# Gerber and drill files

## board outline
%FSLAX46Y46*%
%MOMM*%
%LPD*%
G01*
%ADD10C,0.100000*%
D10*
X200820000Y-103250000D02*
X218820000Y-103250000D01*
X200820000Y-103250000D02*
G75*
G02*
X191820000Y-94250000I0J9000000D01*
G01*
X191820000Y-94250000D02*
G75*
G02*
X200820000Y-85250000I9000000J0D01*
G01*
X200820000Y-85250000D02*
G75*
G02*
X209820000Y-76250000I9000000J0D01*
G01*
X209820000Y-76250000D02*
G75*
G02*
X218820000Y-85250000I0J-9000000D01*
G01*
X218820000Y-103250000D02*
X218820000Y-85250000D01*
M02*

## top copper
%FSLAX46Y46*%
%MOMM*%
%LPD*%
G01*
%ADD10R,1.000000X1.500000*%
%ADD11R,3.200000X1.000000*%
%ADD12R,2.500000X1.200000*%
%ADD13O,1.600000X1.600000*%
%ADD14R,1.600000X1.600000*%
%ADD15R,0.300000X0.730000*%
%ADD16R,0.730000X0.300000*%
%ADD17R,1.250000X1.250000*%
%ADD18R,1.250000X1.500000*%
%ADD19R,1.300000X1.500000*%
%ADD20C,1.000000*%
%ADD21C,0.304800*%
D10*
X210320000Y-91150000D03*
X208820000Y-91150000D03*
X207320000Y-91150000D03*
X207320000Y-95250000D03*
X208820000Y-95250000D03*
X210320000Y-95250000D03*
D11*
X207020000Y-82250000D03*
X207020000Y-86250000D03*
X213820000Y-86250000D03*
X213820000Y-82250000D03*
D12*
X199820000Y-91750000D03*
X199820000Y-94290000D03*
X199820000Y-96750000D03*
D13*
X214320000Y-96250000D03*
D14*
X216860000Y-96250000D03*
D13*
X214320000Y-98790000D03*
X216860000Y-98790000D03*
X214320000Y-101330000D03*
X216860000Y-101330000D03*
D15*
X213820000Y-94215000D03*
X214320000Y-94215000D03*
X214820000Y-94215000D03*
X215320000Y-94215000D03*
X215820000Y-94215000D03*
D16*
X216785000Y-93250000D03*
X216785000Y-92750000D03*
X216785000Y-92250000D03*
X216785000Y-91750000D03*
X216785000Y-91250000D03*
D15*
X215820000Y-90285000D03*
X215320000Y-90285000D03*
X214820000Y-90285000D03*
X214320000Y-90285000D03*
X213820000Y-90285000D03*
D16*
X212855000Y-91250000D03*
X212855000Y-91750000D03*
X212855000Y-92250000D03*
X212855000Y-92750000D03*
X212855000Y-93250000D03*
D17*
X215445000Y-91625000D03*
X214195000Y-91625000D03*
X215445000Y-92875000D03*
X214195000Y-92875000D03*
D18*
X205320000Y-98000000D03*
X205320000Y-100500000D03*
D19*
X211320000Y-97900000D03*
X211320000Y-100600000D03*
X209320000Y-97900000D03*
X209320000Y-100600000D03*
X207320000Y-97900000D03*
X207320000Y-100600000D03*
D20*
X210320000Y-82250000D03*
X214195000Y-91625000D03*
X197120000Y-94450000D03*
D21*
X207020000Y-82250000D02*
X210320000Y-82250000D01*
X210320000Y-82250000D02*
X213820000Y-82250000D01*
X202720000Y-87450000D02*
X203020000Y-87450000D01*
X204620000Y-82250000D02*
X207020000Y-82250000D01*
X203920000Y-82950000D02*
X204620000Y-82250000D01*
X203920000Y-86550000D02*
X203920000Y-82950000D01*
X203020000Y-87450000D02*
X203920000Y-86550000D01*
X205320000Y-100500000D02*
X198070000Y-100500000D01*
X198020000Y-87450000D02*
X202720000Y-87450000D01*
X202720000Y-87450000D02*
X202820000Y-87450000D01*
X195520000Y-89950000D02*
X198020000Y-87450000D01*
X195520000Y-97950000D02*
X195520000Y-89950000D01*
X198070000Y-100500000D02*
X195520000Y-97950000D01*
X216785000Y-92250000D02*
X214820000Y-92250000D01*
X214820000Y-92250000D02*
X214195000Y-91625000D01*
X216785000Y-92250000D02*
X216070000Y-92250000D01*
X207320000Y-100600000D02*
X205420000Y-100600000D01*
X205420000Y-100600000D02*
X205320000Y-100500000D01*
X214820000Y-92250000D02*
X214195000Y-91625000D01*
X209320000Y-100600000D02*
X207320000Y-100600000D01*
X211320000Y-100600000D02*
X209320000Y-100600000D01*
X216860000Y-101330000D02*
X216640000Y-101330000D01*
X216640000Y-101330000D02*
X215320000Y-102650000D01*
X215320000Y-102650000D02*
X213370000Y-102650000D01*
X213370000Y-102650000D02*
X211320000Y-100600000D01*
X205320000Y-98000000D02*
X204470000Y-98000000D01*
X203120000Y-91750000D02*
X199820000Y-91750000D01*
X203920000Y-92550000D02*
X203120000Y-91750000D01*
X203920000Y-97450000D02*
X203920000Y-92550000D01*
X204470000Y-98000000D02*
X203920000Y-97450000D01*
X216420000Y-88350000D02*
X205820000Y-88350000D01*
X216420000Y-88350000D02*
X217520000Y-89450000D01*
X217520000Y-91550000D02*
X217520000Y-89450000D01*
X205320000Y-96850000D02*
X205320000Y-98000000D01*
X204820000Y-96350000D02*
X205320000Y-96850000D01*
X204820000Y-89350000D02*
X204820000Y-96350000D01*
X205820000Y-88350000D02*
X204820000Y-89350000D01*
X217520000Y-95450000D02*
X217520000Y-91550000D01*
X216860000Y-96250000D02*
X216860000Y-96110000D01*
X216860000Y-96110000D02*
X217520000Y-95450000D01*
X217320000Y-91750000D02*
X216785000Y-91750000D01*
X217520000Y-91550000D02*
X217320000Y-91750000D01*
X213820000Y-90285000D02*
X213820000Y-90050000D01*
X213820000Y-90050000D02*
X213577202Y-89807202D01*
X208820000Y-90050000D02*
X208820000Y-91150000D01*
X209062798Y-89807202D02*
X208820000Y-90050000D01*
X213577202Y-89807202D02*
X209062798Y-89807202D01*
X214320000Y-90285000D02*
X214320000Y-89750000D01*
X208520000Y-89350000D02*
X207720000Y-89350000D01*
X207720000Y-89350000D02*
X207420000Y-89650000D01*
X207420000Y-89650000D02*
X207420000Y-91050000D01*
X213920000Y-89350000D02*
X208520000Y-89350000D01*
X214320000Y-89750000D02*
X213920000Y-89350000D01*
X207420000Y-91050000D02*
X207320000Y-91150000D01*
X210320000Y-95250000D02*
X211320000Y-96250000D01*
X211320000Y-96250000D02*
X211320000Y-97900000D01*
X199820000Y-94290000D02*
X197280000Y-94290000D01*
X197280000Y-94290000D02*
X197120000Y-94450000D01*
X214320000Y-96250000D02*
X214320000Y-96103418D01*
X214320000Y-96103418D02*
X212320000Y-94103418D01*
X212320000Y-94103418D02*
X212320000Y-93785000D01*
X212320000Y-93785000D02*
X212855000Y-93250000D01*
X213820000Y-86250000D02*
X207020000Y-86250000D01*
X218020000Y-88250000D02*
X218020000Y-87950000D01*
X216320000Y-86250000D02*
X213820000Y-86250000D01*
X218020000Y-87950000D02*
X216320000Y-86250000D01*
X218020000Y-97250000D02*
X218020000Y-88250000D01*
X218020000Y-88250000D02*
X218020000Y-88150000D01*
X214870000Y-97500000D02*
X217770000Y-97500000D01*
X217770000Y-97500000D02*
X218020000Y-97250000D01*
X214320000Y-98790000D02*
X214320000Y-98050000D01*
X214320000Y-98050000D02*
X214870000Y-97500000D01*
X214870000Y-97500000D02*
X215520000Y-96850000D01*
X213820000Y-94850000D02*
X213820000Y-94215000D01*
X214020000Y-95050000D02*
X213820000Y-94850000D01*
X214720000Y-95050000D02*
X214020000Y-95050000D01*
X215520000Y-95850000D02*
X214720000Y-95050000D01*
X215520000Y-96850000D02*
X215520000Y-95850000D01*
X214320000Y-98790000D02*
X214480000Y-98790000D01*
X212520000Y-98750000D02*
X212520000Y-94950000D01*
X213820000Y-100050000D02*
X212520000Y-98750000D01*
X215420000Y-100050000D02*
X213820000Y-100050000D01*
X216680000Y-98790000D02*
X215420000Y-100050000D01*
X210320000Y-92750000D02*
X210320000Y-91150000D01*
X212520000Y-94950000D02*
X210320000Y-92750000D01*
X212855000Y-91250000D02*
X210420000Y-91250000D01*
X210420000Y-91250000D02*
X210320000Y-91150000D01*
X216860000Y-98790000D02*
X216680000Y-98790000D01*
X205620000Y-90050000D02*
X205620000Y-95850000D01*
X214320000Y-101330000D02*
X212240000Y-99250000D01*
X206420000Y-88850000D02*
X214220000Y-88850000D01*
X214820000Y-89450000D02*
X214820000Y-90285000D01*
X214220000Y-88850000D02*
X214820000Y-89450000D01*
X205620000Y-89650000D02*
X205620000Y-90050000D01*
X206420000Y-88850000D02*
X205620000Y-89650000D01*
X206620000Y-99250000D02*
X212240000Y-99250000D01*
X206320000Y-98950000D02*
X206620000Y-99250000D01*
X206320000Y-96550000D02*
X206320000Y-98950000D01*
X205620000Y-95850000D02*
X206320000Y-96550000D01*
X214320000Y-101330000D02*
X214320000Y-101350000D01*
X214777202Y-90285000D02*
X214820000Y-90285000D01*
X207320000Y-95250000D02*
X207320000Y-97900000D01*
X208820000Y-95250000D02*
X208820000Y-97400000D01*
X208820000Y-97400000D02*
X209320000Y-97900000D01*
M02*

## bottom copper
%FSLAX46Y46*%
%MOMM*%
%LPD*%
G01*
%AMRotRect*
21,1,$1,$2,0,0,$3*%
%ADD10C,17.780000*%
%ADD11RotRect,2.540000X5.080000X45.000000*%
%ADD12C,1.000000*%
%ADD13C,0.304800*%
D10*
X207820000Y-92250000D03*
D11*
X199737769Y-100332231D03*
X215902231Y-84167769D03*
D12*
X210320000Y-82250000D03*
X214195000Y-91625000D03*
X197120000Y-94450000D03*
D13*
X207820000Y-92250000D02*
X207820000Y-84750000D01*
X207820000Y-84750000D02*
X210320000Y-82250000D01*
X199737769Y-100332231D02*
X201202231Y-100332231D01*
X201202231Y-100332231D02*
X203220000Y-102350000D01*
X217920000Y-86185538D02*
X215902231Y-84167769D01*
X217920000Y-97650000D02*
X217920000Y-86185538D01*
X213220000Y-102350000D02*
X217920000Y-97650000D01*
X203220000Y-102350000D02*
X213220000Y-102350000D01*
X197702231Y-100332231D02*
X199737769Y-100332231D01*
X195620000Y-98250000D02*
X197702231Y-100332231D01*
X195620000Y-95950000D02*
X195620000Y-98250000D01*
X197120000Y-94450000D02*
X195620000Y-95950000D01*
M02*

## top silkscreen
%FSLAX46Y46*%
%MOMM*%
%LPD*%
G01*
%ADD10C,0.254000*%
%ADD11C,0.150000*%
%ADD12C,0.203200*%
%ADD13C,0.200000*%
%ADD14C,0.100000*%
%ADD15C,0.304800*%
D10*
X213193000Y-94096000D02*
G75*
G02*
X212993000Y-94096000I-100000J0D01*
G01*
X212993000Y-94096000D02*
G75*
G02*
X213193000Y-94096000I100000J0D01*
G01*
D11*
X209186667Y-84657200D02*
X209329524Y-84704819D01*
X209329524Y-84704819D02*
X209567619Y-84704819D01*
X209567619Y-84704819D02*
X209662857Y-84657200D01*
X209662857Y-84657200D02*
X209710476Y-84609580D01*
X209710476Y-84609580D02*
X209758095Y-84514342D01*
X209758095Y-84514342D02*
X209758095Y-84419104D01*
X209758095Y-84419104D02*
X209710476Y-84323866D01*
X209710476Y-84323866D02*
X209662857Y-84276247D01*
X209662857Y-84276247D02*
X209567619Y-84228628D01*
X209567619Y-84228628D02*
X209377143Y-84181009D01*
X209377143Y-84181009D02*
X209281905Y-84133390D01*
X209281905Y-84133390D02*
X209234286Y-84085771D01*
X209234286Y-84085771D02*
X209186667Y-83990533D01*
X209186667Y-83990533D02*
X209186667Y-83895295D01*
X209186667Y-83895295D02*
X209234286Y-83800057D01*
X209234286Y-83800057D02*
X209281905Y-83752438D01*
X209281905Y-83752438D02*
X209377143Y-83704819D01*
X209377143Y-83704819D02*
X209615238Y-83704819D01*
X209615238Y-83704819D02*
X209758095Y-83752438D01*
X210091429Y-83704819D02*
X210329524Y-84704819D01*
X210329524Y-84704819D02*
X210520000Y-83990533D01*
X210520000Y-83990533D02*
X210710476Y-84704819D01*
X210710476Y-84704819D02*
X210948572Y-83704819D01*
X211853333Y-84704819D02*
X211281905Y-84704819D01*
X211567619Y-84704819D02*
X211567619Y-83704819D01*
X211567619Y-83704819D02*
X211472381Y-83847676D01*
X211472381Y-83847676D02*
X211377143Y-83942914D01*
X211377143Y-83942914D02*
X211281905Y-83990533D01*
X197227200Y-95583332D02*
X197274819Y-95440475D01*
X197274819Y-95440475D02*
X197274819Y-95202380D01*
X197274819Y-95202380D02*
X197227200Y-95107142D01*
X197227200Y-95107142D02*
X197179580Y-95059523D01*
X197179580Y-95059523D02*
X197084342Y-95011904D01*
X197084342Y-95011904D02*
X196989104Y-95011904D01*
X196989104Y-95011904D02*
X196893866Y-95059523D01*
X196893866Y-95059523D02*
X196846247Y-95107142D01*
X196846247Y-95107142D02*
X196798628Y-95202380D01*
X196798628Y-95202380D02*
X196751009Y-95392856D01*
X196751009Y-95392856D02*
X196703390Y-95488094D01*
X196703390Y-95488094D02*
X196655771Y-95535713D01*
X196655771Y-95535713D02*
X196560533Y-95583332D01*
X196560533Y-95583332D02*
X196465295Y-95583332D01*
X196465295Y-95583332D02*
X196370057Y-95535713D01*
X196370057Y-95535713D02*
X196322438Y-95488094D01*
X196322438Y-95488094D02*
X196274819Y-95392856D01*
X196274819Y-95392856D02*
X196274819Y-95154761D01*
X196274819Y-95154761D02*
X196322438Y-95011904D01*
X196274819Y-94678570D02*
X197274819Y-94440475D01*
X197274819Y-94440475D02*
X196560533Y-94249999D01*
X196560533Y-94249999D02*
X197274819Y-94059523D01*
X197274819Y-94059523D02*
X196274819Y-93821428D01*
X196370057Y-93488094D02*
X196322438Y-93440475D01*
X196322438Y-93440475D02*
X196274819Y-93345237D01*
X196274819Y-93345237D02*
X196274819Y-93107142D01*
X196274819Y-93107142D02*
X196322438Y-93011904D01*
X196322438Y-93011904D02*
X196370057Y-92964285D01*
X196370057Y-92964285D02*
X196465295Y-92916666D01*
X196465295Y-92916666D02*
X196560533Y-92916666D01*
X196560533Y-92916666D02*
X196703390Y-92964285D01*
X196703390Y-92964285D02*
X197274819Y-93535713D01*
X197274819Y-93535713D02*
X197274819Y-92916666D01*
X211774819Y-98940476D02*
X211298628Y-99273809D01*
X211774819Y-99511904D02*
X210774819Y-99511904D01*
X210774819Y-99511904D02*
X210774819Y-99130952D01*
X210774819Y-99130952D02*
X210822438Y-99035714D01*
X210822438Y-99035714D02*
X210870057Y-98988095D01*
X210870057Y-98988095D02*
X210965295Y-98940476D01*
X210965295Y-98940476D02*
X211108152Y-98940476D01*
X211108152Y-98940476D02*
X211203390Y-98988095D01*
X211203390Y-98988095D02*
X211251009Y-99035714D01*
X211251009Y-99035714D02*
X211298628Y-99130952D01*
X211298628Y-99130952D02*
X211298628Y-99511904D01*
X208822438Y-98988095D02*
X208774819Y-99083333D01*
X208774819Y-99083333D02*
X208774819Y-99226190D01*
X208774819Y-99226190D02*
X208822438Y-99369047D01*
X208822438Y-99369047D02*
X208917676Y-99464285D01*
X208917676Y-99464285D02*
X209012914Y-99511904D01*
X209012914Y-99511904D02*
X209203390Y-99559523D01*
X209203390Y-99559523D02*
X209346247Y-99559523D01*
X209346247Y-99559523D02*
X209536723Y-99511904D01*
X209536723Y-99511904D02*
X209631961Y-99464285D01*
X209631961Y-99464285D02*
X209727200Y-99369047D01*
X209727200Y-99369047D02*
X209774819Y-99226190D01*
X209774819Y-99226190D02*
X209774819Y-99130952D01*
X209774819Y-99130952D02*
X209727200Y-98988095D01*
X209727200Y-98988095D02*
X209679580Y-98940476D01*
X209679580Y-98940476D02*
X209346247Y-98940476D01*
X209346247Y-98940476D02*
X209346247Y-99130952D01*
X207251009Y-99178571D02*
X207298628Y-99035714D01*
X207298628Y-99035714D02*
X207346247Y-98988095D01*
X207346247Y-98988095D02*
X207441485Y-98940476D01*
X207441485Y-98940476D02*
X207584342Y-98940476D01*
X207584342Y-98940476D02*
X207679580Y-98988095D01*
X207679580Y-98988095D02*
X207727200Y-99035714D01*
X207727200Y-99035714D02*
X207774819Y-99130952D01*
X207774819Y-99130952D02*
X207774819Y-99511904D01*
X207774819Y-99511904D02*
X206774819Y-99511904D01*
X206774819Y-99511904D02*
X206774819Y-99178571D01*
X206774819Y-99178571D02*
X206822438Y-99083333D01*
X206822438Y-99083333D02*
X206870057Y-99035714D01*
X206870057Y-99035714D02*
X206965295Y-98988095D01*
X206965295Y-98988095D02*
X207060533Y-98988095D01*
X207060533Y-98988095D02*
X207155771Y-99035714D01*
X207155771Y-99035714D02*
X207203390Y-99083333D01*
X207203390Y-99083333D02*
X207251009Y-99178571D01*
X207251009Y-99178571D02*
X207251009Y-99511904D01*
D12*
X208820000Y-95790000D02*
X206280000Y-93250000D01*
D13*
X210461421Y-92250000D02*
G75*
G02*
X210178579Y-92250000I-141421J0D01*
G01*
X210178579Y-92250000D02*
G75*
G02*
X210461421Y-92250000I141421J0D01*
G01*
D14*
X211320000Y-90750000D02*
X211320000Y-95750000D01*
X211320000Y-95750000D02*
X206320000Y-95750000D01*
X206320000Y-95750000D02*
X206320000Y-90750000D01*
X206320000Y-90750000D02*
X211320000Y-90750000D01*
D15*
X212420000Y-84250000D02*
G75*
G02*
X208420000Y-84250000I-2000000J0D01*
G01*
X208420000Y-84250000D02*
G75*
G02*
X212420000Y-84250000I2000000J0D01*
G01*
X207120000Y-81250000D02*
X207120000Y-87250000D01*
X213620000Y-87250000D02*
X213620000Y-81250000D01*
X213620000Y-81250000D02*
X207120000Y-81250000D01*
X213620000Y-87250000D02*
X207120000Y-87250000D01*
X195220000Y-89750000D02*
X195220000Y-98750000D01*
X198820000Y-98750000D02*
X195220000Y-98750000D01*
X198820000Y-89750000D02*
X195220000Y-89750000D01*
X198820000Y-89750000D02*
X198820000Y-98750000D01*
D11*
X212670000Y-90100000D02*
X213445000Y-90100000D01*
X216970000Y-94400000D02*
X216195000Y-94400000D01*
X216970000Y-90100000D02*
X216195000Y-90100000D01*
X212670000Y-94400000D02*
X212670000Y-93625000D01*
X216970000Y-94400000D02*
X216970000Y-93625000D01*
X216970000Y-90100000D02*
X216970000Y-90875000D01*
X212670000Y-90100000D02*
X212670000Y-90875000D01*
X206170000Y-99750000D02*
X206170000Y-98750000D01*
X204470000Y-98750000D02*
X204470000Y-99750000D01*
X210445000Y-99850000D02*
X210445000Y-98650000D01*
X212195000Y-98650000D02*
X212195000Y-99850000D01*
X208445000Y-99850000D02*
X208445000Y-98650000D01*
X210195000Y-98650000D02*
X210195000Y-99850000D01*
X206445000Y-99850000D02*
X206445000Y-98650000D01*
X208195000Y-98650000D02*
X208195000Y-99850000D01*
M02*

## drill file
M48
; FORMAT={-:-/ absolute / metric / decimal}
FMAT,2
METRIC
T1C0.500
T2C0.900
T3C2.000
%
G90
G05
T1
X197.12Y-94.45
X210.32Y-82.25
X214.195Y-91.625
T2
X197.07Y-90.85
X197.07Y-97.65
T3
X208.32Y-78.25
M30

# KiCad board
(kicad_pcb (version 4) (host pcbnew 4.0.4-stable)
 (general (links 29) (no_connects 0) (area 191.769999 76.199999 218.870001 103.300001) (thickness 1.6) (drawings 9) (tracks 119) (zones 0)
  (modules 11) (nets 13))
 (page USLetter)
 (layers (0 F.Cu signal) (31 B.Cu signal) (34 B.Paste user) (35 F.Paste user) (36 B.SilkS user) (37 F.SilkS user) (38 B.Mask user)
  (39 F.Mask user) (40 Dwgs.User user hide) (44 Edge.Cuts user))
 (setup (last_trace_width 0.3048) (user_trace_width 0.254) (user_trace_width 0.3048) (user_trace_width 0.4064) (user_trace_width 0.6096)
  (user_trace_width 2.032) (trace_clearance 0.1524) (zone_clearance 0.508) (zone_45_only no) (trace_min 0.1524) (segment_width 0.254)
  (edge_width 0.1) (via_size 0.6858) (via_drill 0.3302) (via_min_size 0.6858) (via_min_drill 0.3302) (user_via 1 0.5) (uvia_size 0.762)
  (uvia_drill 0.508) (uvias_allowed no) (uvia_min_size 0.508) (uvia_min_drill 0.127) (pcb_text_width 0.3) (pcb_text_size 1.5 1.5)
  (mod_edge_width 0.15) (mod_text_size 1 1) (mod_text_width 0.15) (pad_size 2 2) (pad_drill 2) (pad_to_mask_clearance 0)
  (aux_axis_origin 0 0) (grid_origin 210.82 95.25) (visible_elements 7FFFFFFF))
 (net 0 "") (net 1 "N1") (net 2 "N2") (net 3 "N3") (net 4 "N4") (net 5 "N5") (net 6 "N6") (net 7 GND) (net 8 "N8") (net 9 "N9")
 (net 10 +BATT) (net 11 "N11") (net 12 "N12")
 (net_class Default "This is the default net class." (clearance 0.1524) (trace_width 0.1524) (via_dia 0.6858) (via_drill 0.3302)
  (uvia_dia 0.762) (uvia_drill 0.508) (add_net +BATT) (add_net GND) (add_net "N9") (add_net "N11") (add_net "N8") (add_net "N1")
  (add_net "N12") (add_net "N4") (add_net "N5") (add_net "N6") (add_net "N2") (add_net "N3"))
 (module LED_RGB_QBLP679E (layer F.Cu) (at 208.82 93.25 270)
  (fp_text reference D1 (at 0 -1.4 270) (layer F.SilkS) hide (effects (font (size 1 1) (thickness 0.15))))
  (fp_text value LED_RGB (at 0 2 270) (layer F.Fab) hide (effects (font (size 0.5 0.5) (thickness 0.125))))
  (fp_line (start 2.54 0) (end 0 2.54) (layer F.SilkS) (width 0.2032))
  (fp_circle (center -1 -1.5) (end -1.1 -1.6) (layer F.SilkS) (width 0.2))
  (fp_line (start -2.5 -2.5) (end 2.5 -2.5) (layer F.SilkS) (width 0.1))
  (fp_line (start 2.5 -2.5) (end 2.5 2.5) (layer F.SilkS) (width 0.1))
  (fp_line (start 2.5 2.5) (end -2.5 2.5) (layer F.SilkS) (width 0.1))
  (fp_line (start -2.5 2.5) (end -2.5 -2.5) (layer F.SilkS) (width 0.1))
  (pad 4 smd rect (at -2.1 -1.5) (size 1 1.5) (layers F.Cu F.Paste F.Mask) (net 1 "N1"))
  (pad 5 smd rect (at -2.1 0) (size 1 1.5) (layers F.Cu F.Paste F.Mask) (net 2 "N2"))
  (pad 6 smd rect (at -2.1 1.5) (size 1 1.5) (layers F.Cu F.Paste F.Mask) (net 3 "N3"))
  (pad 1 smd rect (at 2 1.5) (size 1 1.5) (layers F.Cu F.Paste F.Mask) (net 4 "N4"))
  (pad 2 smd rect (at 2 0) (size 1 1.5) (layers F.Cu F.Paste F.Mask) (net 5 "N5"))
  (pad 3 smd rect (at 2 -1.5) (size 1 1.5) (layers F.Cu F.Paste F.Mask) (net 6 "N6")))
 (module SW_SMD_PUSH (layer F.Cu) (at 213.82 86.25 180)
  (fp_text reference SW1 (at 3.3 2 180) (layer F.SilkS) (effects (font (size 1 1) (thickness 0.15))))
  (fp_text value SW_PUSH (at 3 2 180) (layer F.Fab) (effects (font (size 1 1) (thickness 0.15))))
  (fp_circle (center 3.4 2) (end 3.4 0) (layer F.SilkS) (width 0.3048))
  (fp_line (start 6.7 5) (end 6.7 -1) (layer F.SilkS) (width 0.3048))
  (fp_line (start 0.2 -1) (end 0.2 5) (layer F.SilkS) (width 0.3048))
  (fp_line (start 0.2 5) (end 6.7 5) (layer F.SilkS) (width 0.3048))
  (fp_line (start 0.2 -1) (end 6.7 -1) (layer F.SilkS) (width 0.3048))
  (pad 2 smd rect (at 6.8 4 180) (size 3.2 1) (layers F.Cu F.Paste F.Mask) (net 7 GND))
  (pad 1 smd rect (at 6.8 0 180) (size 3.2 1) (layers F.Cu F.Paste F.Mask) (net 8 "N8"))
  (pad 1 smd rect (at 0 0 180) (size 3.2 1) (layers F.Cu F.Paste F.Mask) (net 8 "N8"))
  (pad 2 smd rect (at 0 4 180) (size 3.2 1) (layers F.Cu F.Paste F.Mask) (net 7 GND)))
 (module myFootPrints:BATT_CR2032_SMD (layer B.Cu) (at 207.82 92.25 45)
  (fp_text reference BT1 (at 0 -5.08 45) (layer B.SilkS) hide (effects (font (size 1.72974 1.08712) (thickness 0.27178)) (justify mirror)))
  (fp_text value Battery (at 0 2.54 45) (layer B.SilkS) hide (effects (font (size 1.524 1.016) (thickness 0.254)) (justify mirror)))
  (pad 2 smd circle (at 0 0 45) (size 17.78 17.78) (layers B.Cu B.Paste B.Mask) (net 7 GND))
  (pad 1 smd rect (at -11.43 0 45) (size 2.54 5.08) (layers B.Cu B.Paste B.Mask) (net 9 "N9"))
  (pad 1 smd rect (at 11.43 0 45) (size 2.54 5.08) (layers B.Cu B.Paste B.Mask) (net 9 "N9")))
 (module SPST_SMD (layer F.Cu) (at 199.82 94.25 270)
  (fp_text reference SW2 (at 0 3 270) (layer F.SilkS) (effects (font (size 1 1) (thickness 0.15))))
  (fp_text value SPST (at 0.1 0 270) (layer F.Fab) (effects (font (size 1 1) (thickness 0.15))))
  (fp_line (start -4.5 4.6) (end 4.5 4.6) (layer F.SilkS) (width 0.3048))
  (fp_line (start 4.5 1) (end 4.5 4.6) (layer F.SilkS) (width 0.3048))
  (fp_line (start -4.5 1) (end -4.5 4.6) (layer F.SilkS) (width 0.3048))
  (fp_line (start -4.5 1) (end 4.5 1) (layer F.SilkS) (width 0.3048))
  (pad "" np_thru_hole circle (at 3.4 2.75 270) (size 0.9 0.9) (drill 0.9) (layers *.Cu *.Mask))
  (pad 1 smd rect (at -2.5 0 270) (size 1.2 2.5) (layers F.Cu F.Paste F.Mask) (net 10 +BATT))
  (pad 2 smd rect (at 0.04 0 270) (size 1.2 2.5) (layers F.Cu F.Paste F.Mask) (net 9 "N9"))
  (pad 3 smd rect (at 2.5 0 270) (size 1.2 2.5) (layers F.Cu F.Paste F.Mask))
  (pad "" np_thru_hole circle (at -3.4 2.75 270) (size 0.9 0.9) (drill 0.9) (layers *.Cu *.Mask)))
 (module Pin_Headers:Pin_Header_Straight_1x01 (layer F.Cu) (at 208.32 78.25)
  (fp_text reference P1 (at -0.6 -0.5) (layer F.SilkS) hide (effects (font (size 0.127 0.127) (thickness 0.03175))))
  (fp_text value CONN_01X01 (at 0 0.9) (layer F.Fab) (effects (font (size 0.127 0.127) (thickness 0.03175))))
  (pad "" np_thru_hole circle (at 0 0) (size 2 2) (drill 2) (layers *.Cu *.Mask)))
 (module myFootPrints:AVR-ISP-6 (layer F.Cu) (at 214.32 96.25)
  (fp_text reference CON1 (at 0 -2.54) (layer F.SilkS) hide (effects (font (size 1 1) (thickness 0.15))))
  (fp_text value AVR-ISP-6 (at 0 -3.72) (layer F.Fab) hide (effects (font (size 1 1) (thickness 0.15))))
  (pad 1 smd oval (at 0 0) (size 1.6 1.6) (layers F.Cu F.Paste F.Mask) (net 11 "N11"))
  (pad 2 smd rect (at 2.54 0) (size 1.6 1.6) (layers F.Cu F.Paste F.Mask) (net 10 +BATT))
  (pad 3 smd oval (at 0 2.54) (size 1.6 1.6) (layers F.Cu F.Paste F.Mask) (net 8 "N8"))
  (pad 4 smd oval (at 2.54 2.54) (size 1.6 1.6) (layers F.Cu F.Paste F.Mask) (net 1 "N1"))
  (pad 5 smd oval (at 0 5.08) (size 1.6 1.6) (layers F.Cu F.Paste F.Mask) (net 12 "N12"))
  (pad 6 smd oval (at 2.54 5.08) (size 1.6 1.6) (layers F.Cu F.Paste F.Mask) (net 7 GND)))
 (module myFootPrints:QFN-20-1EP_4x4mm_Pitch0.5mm (layer F.Cu) (at 214.82 92.25 90)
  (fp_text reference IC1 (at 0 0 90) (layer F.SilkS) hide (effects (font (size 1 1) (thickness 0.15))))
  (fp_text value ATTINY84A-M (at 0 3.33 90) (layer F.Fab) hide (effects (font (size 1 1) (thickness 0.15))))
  (fp_line (start 2.15 -2.15) (end 2.15 -1.375) (layer F.SilkS) (width 0.15))
  (fp_line (start -2.15 2.15) (end -2.15 1.375) (layer F.SilkS) (width 0.15))
  (fp_line (start 2.15 2.15) (end 2.15 1.375) (layer F.SilkS) (width 0.15))
  (fp_line (start -2.15 -2.15) (end -1.375 -2.15) (layer F.SilkS) (width 0.15))
  (fp_line (start -2.15 2.15) (end -1.375 2.15) (layer F.SilkS) (width 0.15))
  (fp_line (start 2.15 2.15) (end 1.375 2.15) (layer F.SilkS) (width 0.15))
  (fp_line (start 2.15 -2.15) (end 1.375 -2.15) (layer F.SilkS) (width 0.15))
  (pad 1 smd rect (at -1.965 -1 90) (size 0.73 0.3) (layers F.Cu F.Paste F.Mask) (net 8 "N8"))
  (pad 2 smd rect (at -1.965 -0.5 90) (size 0.73 0.3) (layers F.Cu F.Paste F.Mask))
  (pad 3 smd rect (at -1.965 0 90) (size 0.73 0.3) (layers F.Cu F.Paste F.Mask))
  (pad 4 smd rect (at -1.965 0.5 90) (size 0.73 0.3) (layers F.Cu F.Paste F.Mask))
  (pad 5 smd rect (at -1.965 1 90) (size 0.73 0.3) (layers F.Cu F.Paste F.Mask))
  (pad 6 smd rect (at -1 1.965 180) (size 0.73 0.3) (layers F.Cu F.Paste F.Mask))
  (pad 7 smd rect (at -0.5 1.965 180) (size 0.73 0.3) (layers F.Cu F.Paste F.Mask))
  (pad 8 smd rect (at 0 1.965 180) (size 0.73 0.3) (layers F.Cu F.Paste F.Mask) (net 7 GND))
  (pad 9 smd rect (at 0.5 1.965 180) (size 0.73 0.3) (layers F.Cu F.Paste F.Mask) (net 10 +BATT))
  (pad 10 smd rect (at 1 1.965 180) (size 0.73 0.3) (layers F.Cu F.Paste F.Mask))
  (pad 11 smd rect (at 1.965 1 90) (size 0.73 0.3) (layers F.Cu F.Paste F.Mask))
  (pad 12 smd rect (at 1.965 0.5 90) (size 0.73 0.3) (layers F.Cu F.Paste F.Mask))
  (pad 13 smd rect (at 1.965 0 90) (size 0.73 0.3) (layers F.Cu F.Paste F.Mask) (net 12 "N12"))
  (pad 14 smd rect (at 1.965 -0.5 90) (size 0.73 0.3) (layers F.Cu F.Paste F.Mask) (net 3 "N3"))
  (pad 15 smd rect (at 1.965 -1 90) (size 0.73 0.3) (layers F.Cu F.Paste F.Mask) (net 2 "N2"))
  (pad 16 smd rect (at 1 -1.965 180) (size 0.73 0.3) (layers F.Cu F.Paste F.Mask) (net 1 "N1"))
  (pad 17 smd rect (at 0.5 -1.965 180) (size 0.73 0.3) (layers F.Cu F.Paste F.Mask))
  (pad 18 smd rect (at 0 -1.965 180) (size 0.73 0.3) (layers F.Cu F.Paste F.Mask))
  (pad 19 smd rect (at -0.5 -1.965 180) (size 0.73 0.3) (layers F.Cu F.Paste F.Mask))
  (pad 20 smd rect (at -1 -1.965 180) (size 0.73 0.3) (layers F.Cu F.Paste F.Mask) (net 11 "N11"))
  (pad 8 smd rect (at 0.625 0.625 90) (size 1.25 1.25) (layers F.Cu F.Paste F.Mask) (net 7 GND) (solder_paste_margin_ratio -0.2))
  (pad 8 smd rect (at 0.625 -0.625 90) (size 1.25 1.25) (layers F.Cu F.Paste F.Mask) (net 7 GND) (solder_paste_margin_ratio -0.2))
  (pad 8 smd rect (at -0.625 0.625 90) (size 1.25 1.25) (layers F.Cu F.Paste F.Mask) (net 7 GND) (solder_paste_margin_ratio -0.2))
  (pad 8 smd rect (at -0.625 -0.625 90) (size 1.25 1.25) (layers F.Cu F.Paste F.Mask) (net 7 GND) (solder_paste_margin_ratio -0.2)))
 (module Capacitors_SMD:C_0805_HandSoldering (layer F.Cu) (at 205.32 99.25 270)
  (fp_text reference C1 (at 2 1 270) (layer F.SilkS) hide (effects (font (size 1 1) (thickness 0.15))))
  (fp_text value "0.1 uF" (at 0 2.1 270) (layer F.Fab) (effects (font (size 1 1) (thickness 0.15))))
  (fp_line (start 0.5 -0.85) (end -0.5 -0.85) (layer F.SilkS) (width 0.15))
  (fp_line (start -0.5 0.85) (end 0.5 0.85) (layer F.SilkS) (width 0.15))
  (pad 1 smd rect (at -1.25 0 270) (size 1.5 1.25) (layers F.Cu F.Paste F.Mask) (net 10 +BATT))
  (pad 2 smd rect (at 1.25 0 270) (size 1.5 1.25) (layers F.Cu F.Paste F.Mask) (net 7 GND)))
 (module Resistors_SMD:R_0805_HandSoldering (layer F.Cu) (at 211.32 99.25 270)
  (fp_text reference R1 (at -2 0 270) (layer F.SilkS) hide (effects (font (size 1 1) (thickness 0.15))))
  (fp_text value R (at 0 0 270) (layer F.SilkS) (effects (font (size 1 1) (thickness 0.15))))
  (fp_line (start 0.6 0.875) (end -0.6 0.875) (layer F.SilkS) (width 0.15))
  (fp_line (start -0.6 -0.875) (end 0.6 -0.875) (layer F.SilkS) (width 0.15))
  (pad 1 smd rect (at -1.35 0 270) (size 1.5 1.3) (layers F.Cu F.Paste F.Mask) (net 6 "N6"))
  (pad 2 smd rect (at 1.35 0 270) (size 1.5 1.3) (layers F.Cu F.Paste F.Mask) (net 7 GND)))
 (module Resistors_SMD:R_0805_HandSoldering (layer F.Cu) (at 209.32 99.25 270)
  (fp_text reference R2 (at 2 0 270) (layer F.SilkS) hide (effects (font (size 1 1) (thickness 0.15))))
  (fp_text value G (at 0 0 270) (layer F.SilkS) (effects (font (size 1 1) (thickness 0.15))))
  (fp_line (start 0.6 0.875) (end -0.6 0.875) (layer F.SilkS) (width 0.15))
  (fp_line (start -0.6 -0.875) (end 0.6 -0.875) (layer F.SilkS) (width 0.15))
  (pad 1 smd rect (at -1.35 0 270) (size 1.5 1.3) (layers F.Cu F.Paste F.Mask) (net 5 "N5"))
  (pad 2 smd rect (at 1.35 0 270) (size 1.5 1.3) (layers F.Cu F.Paste F.Mask) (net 7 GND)))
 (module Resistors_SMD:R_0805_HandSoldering (layer F.Cu) (at 207.32 99.25 270)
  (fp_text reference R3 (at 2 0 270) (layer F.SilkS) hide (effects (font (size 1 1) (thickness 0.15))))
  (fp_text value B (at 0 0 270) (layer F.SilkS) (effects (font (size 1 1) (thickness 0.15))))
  (fp_line (start 0.6 0.875) (end -0.6 0.875) (layer F.SilkS) (width 0.15))
  (fp_line (start -0.6 -0.875) (end 0.6 -0.875) (layer F.SilkS) (width 0.15))
  (pad 1 smd rect (at -1.35 0 270) (size 1.5 1.3) (layers F.Cu F.Paste F.Mask) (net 4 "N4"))
  (pad 2 smd rect (at 1.35 0 270) (size 1.5 1.3) (layers F.Cu F.Paste F.Mask) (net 7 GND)))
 (gr_circle (center 213.093 94.096) (end 213.193 94.096) (layer F.SilkS) (width 0.254))
 (gr_line (start 200.82 103.25) (end 218.82 103.25) (angle 90) (layer Edge.Cuts) (width 0.1))
 (gr_arc (start 200.82 94.25) (end 200.82 103.25) (angle 90) (layer Edge.Cuts) (width 0.1))
 (gr_arc (start 200.82 94.25) (end 191.82 94.25) (angle 90) (layer Edge.Cuts) (width 0.1))
 (gr_arc (start 209.82 85.25) (end 200.82 85.25) (angle 90) (layer Edge.Cuts) (width 0.1))
 (gr_arc (start 209.82 85.25) (end 209.82 76.25) (angle 90) (layer Edge.Cuts) (width 0.1))
 (gr_line (start 218.82 103.25) (end 218.82 85.25) (angle 90) (layer Edge.Cuts) (width 0.1))
 (segment (start 207.02 82.25) (end 210.32 82.25) (width 0.3048) (layer F.Cu) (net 7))
 (segment (start 207.82 92.25) (end 207.82 84.75) (width 0.3048) (layer B.Cu) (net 7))
 (segment (start 207.82 84.75) (end 210.32 82.25) (width 0.3048) (layer B.Cu) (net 7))
 (via (at 210.32 82.25) (size 1) (drill 0.5) (layers F.Cu B.Cu) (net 7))
 (segment (start 210.32 82.25) (end 213.82 82.25) (width 0.3048) (layer F.Cu) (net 7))
 (segment (start 202.72 87.45) (end 203.02 87.45) (width 0.3048) (layer F.Cu) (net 7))
 (segment (start 204.62 82.25) (end 207.02 82.25) (width 0.3048) (layer F.Cu) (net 7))
 (segment (start 203.92 82.95) (end 204.62 82.25) (width 0.3048) (layer F.Cu) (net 7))
 (segment (start 203.92 86.55) (end 203.92 82.95) (width 0.3048) (layer F.Cu) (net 7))
 (segment (start 203.02 87.45) (end 203.92 86.55) (width 0.3048) (layer F.Cu) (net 7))
 (segment (start 205.32 100.5) (end 198.07 100.5) (width 0.3048) (layer F.Cu) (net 7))
 (segment (start 198.02 87.45) (end 202.72 87.45) (width 0.3048) (layer F.Cu) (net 7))
 (segment (start 202.72 87.45) (end 202.82 87.45) (width 0.3048) (layer F.Cu) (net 7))
 (segment (start 195.52 89.95) (end 198.02 87.45) (width 0.3048) (layer F.Cu) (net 7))
 (segment (start 195.52 97.95) (end 195.52 89.95) (width 0.3048) (layer F.Cu) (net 7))
 (segment (start 198.07 100.5) (end 195.52 97.95) (width 0.3048) (layer F.Cu) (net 7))
 (segment (start 216.785 92.25) (end 214.82 92.25) (width 0.3048) (layer F.Cu) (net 7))
 (segment (start 214.82 92.25) (end 214.195 91.625) (width 0.3048) (layer F.Cu) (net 7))
 (via (at 214.195 91.625) (size 1) (drill 0.5) (layers F.Cu B.Cu) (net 7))
 (segment (start 216.785 92.25) (end 216.07 92.25) (width 0.3048) (layer F.Cu) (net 7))
 (segment (start 207.32 100.6) (end 205.42 100.6) (width 0.3048) (layer F.Cu) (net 7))
 (segment (start 205.42 100.6) (end 205.32 100.5) (width 0.3048) (layer F.Cu) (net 7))
 (segment (start 214.82 92.25) (end 214.195 91.625) (width 0.3048) (layer F.Cu) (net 7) (status 30))
 (segment (start 209.32 100.6) (end 207.32 100.6) (width 0.3048) (layer F.Cu) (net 7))
 (segment (start 211.32 100.6) (end 209.32 100.6) (width 0.3048) (layer F.Cu) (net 7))
 (segment (start 216.86 101.33) (end 216.64 101.33) (width 0.3048) (layer F.Cu) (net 7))
 (segment (start 216.64 101.33) (end 215.32 102.65) (width 0.3048) (layer F.Cu) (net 7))
 (segment (start 215.32 102.65) (end 213.37 102.65) (width 0.3048) (layer F.Cu) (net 7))
 (segment (start 213.37 102.65) (end 211.32 100.6) (width 0.3048) (layer F.Cu) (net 7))
 (segment (start 205.32 98) (end 204.47 98) (width 0.3048) (layer F.Cu) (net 10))
 (segment (start 203.12 91.75) (end 199.82 91.75) (width 0.3048) (layer F.Cu) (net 10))
 (segment (start 203.92 92.55) (end 203.12 91.75) (width 0.3048) (layer F.Cu) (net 10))
 (segment (start 203.92 97.45) (end 203.92 92.55) (width 0.3048) (layer F.Cu) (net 10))
 (segment (start 204.47 98) (end 203.92 97.45) (width 0.3048) (layer F.Cu) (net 10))
 (segment (start 216.42 88.35) (end 205.82 88.35) (width 0.3048) (layer F.Cu) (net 10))
 (segment (start 216.42 88.35) (end 217.52 89.45) (width 0.3048) (layer F.Cu) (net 10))
 (segment (start 217.52 91.55) (end 217.52 89.45) (width 0.3048) (layer F.Cu) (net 10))
 (segment (start 205.32 96.85) (end 205.32 98) (width 0.3048) (layer F.Cu) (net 10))
 (segment (start 204.82 96.35) (end 205.32 96.85) (width 0.3048) (layer F.Cu) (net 10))
 (segment (start 204.82 89.35) (end 204.82 96.35) (width 0.3048) (layer F.Cu) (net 10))
 (segment (start 205.82 88.35) (end 204.82 89.35) (width 0.3048) (layer F.Cu) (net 10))
 (segment (start 217.52 95.45) (end 217.52 91.55) (width 0.3048) (layer F.Cu) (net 10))
 (segment (start 216.86 96.25) (end 216.86 96.11) (width 0.3048) (layer F.Cu) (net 10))
 (segment (start 216.86 96.11) (end 217.52 95.45) (width 0.3048) (layer F.Cu) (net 10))
 (segment (start 217.32 91.75) (end 216.785 91.75) (width 0.3048) (layer F.Cu) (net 10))
 (segment (start 217.52 91.55) (end 217.32 91.75) (width 0.3048) (layer F.Cu) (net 10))
 (segment (start 213.82 90.285) (end 213.82 90.05) (width 0.3048) (layer F.Cu) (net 2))
 (segment (start 213.82 90.05) (end 213.577202 89.807202) (width 0.3048) (layer F.Cu) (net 2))
 (segment (start 208.82 90.05) (end 208.82 91.15) (width 0.3048) (layer F.Cu) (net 2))
 (segment (start 209.062798 89.807202) (end 208.82 90.05) (width 0.3048) (layer F.Cu) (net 2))
 (segment (start 213.577202 89.807202) (end 209.062798 89.807202) (width 0.3048) (layer F.Cu) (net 2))
 (segment (start 214.32 90.285) (end 214.32 89.75) (width 0.3048) (layer F.Cu) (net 3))
 (segment (start 208.52 89.35) (end 207.72 89.35) (width 0.3048) (layer F.Cu) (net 3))
 (segment (start 207.72 89.35) (end 207.42 89.65) (width 0.3048) (layer F.Cu) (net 3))
 (segment (start 207.42 89.65) (end 207.42 91.05) (width 0.3048) (layer F.Cu) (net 3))
 (segment (start 213.92 89.35) (end 208.52 89.35) (width 0.3048) (layer F.Cu) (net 3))
 (segment (start 214.32 89.75) (end 213.92 89.35) (width 0.3048) (layer F.Cu) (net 3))
 (segment (start 207.42 91.05) (end 207.32 91.15) (width 0.3048) (layer F.Cu) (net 3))
 (segment (start 210.32 95.25) (end 211.32 96.25) (width 0.3048) (layer F.Cu) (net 6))
 (segment (start 211.32 96.25) (end 211.32 97.9) (width 0.3048) (layer F.Cu) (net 6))
 (segment (start 199.737769 100.332231) (end 201.202231 100.332231) (width 0.3048) (layer B.Cu) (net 9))
 (segment (start 201.202231 100.332231) (end 203.22 102.35) (width 0.3048) (layer B.Cu) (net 9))
 (segment (start 217.92 86.185538) (end 215.902231 84.167769) (width 0.3048) (layer B.Cu) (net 9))
 (segment (start 217.92 97.65) (end 217.92 86.185538) (width 0.3048) (layer B.Cu) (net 9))
 (segment (start 213.22 102.35) (end 217.92 97.65) (width 0.3048) (layer B.Cu) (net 9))
 (segment (start 203.22 102.35) (end 213.22 102.35) (width 0.3048) (layer B.Cu) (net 9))
 (segment (start 199.82 94.29) (end 197.28 94.29) (width 0.3048) (layer F.Cu) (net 9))
 (segment (start 197.702231 100.332231) (end 199.737769 100.332231) (width 0.3048) (layer B.Cu) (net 9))
 (segment (start 195.62 98.25) (end 197.702231 100.332231) (width 0.3048) (layer B.Cu) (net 9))
 (segment (start 195.62 95.95) (end 195.62 98.25) (width 0.3048) (layer B.Cu) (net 9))
 (segment (start 197.12 94.45) (end 195.62 95.95) (width 0.3048) (layer B.Cu) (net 9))
 (via (at 197.12 94.45) (size 1) (drill 0.5) (layers F.Cu B.Cu) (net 9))
 (segment (start 197.28 94.29) (end 197.12 94.45) (width 0.3048) (layer F.Cu) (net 9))
 (segment (start 214.32 96.25) (end 214.32 96.103418) (width 0.3048) (layer F.Cu) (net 11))
 (segment (start 214.32 96.103418) (end 212.32 94.103418) (width 0.3048) (layer F.Cu) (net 11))
 (segment (start 212.32 94.103418) (end 212.32 93.785) (width 0.3048) (layer F.Cu) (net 11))
 (segment (start 212.32 93.785) (end 212.855 93.25) (width 0.3048) (layer F.Cu) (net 11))
 (segment (start 213.82 86.25) (end 207.02 86.25) (width 0.3048) (layer F.Cu) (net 8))
 (segment (start 218.02 88.25) (end 218.02 87.95) (width 0.3048) (layer F.Cu) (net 8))
 (segment (start 216.32 86.25) (end 213.82 86.25) (width 0.3048) (layer F.Cu) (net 8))
 (segment (start 218.02 87.95) (end 216.32 86.25) (width 0.3048) (layer F.Cu) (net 8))
 (segment (start 218.02 97.25) (end 218.02 88.25) (width 0.3048) (layer F.Cu) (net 8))
 (segment (start 218.02 88.25) (end 218.02 88.15) (width 0.3048) (layer F.Cu) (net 8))
 (segment (start 214.87 97.5) (end 217.77 97.5) (width 0.3048) (layer F.Cu) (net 8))
 (segment (start 217.77 97.5) (end 218.02 97.25) (width 0.3048) (layer F.Cu) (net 8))
 (segment (start 214.32 98.79) (end 214.32 98.05) (width 0.3048) (layer F.Cu) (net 8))
 (segment (start 214.32 98.05) (end 214.87 97.5) (width 0.3048) (layer F.Cu) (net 8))
 (segment (start 214.87 97.5) (end 215.52 96.85) (width 0.3048) (layer F.Cu) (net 8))
 (segment (start 213.82 94.85) (end 213.82 94.215) (width 0.3048) (layer F.Cu) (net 8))
 (segment (start 214.02 95.05) (end 213.82 94.85) (width 0.3048) (layer F.Cu) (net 8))
 (segment (start 214.72 95.05) (end 214.02 95.05) (width 0.3048) (layer F.Cu) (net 8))
 (segment (start 215.52 95.85) (end 214.72 95.05) (width 0.3048) (layer F.Cu) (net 8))
 (segment (start 215.52 96.85) (end 215.52 95.85) (width 0.3048) (layer F.Cu) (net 8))
 (segment (start 214.32 98.79) (end 214.48 98.79) (width 0.3048) (layer F.Cu) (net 8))
 (segment (start 212.52 98.75) (end 212.52 94.95) (width 0.3048) (layer F.Cu) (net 1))
 (segment (start 213.82 100.05) (end 212.52 98.75) (width 0.3048) (layer F.Cu) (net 1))
 (segment (start 215.42 100.05) (end 213.82 100.05) (width 0.3048) (layer F.Cu) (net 1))
 (segment (start 216.68 98.79) (end 215.42 100.05) (width 0.3048) (layer F.Cu) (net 1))
 (segment (start 210.32 92.75) (end 210.32 91.15) (width 0.3048) (layer F.Cu) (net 1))
 (segment (start 212.52 94.95) (end 210.32 92.75) (width 0.3048) (layer F.Cu) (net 1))
 (segment (start 212.855 91.25) (end 210.42 91.25) (width 0.3048) (layer F.Cu) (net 1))
 (segment (start 210.42 91.25) (end 210.32 91.15) (width 0.3048) (layer F.Cu) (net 1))
 (segment (start 216.86 98.79) (end 216.68 98.79) (width 0.3048) (layer F.Cu) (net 1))
 (segment (start 205.62 90.05) (end 205.62 95.85) (width 0.3048) (layer F.Cu) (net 12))
 (segment (start 214.32 101.33) (end 212.24 99.25) (width 0.3048) (layer F.Cu) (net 12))
 (segment (start 206.42 88.85) (end 214.22 88.85) (width 0.3048) (layer F.Cu) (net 12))
 (segment (start 214.82 89.45) (end 214.82 90.285) (width 0.3048) (layer F.Cu) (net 12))
 (segment (start 214.22 88.85) (end 214.82 89.45) (width 0.3048) (layer F.Cu) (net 12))
 (segment (start 205.62 89.65) (end 205.62 90.05) (width 0.3048) (layer F.Cu) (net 12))
 (segment (start 206.42 88.85) (end 205.62 89.65) (width 0.3048) (layer F.Cu) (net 12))
 (segment (start 206.62 99.25) (end 212.24 99.25) (width 0.3048) (layer F.Cu) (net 12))
 (segment (start 206.32 98.95) (end 206.62 99.25) (width 0.3048) (layer F.Cu) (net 12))
 (segment (start 206.32 96.55) (end 206.32 98.95) (width 0.3048) (layer F.Cu) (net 12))
 (segment (start 205.62 95.85) (end 206.32 96.55) (width 0.3048) (layer F.Cu) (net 12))
 (segment (start 214.32 101.33) (end 214.32 101.35) (width 0.3048) (layer F.Cu) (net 12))
 (segment (start 214.777202 90.285) (end 214.82 90.285) (width 0.3048) (layer F.Cu) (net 12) (status 30))
 (segment (start 207.32 95.25) (end 207.32 97.9) (width 0.3048) (layer F.Cu) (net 4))
 (segment (start 208.82 95.25) (end 208.82 97.4) (width 0.3048) (layer F.Cu) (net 5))
 (segment (start 208.82 97.4) (end 209.32 97.9) (width 0.3048) (layer F.Cu) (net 5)))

